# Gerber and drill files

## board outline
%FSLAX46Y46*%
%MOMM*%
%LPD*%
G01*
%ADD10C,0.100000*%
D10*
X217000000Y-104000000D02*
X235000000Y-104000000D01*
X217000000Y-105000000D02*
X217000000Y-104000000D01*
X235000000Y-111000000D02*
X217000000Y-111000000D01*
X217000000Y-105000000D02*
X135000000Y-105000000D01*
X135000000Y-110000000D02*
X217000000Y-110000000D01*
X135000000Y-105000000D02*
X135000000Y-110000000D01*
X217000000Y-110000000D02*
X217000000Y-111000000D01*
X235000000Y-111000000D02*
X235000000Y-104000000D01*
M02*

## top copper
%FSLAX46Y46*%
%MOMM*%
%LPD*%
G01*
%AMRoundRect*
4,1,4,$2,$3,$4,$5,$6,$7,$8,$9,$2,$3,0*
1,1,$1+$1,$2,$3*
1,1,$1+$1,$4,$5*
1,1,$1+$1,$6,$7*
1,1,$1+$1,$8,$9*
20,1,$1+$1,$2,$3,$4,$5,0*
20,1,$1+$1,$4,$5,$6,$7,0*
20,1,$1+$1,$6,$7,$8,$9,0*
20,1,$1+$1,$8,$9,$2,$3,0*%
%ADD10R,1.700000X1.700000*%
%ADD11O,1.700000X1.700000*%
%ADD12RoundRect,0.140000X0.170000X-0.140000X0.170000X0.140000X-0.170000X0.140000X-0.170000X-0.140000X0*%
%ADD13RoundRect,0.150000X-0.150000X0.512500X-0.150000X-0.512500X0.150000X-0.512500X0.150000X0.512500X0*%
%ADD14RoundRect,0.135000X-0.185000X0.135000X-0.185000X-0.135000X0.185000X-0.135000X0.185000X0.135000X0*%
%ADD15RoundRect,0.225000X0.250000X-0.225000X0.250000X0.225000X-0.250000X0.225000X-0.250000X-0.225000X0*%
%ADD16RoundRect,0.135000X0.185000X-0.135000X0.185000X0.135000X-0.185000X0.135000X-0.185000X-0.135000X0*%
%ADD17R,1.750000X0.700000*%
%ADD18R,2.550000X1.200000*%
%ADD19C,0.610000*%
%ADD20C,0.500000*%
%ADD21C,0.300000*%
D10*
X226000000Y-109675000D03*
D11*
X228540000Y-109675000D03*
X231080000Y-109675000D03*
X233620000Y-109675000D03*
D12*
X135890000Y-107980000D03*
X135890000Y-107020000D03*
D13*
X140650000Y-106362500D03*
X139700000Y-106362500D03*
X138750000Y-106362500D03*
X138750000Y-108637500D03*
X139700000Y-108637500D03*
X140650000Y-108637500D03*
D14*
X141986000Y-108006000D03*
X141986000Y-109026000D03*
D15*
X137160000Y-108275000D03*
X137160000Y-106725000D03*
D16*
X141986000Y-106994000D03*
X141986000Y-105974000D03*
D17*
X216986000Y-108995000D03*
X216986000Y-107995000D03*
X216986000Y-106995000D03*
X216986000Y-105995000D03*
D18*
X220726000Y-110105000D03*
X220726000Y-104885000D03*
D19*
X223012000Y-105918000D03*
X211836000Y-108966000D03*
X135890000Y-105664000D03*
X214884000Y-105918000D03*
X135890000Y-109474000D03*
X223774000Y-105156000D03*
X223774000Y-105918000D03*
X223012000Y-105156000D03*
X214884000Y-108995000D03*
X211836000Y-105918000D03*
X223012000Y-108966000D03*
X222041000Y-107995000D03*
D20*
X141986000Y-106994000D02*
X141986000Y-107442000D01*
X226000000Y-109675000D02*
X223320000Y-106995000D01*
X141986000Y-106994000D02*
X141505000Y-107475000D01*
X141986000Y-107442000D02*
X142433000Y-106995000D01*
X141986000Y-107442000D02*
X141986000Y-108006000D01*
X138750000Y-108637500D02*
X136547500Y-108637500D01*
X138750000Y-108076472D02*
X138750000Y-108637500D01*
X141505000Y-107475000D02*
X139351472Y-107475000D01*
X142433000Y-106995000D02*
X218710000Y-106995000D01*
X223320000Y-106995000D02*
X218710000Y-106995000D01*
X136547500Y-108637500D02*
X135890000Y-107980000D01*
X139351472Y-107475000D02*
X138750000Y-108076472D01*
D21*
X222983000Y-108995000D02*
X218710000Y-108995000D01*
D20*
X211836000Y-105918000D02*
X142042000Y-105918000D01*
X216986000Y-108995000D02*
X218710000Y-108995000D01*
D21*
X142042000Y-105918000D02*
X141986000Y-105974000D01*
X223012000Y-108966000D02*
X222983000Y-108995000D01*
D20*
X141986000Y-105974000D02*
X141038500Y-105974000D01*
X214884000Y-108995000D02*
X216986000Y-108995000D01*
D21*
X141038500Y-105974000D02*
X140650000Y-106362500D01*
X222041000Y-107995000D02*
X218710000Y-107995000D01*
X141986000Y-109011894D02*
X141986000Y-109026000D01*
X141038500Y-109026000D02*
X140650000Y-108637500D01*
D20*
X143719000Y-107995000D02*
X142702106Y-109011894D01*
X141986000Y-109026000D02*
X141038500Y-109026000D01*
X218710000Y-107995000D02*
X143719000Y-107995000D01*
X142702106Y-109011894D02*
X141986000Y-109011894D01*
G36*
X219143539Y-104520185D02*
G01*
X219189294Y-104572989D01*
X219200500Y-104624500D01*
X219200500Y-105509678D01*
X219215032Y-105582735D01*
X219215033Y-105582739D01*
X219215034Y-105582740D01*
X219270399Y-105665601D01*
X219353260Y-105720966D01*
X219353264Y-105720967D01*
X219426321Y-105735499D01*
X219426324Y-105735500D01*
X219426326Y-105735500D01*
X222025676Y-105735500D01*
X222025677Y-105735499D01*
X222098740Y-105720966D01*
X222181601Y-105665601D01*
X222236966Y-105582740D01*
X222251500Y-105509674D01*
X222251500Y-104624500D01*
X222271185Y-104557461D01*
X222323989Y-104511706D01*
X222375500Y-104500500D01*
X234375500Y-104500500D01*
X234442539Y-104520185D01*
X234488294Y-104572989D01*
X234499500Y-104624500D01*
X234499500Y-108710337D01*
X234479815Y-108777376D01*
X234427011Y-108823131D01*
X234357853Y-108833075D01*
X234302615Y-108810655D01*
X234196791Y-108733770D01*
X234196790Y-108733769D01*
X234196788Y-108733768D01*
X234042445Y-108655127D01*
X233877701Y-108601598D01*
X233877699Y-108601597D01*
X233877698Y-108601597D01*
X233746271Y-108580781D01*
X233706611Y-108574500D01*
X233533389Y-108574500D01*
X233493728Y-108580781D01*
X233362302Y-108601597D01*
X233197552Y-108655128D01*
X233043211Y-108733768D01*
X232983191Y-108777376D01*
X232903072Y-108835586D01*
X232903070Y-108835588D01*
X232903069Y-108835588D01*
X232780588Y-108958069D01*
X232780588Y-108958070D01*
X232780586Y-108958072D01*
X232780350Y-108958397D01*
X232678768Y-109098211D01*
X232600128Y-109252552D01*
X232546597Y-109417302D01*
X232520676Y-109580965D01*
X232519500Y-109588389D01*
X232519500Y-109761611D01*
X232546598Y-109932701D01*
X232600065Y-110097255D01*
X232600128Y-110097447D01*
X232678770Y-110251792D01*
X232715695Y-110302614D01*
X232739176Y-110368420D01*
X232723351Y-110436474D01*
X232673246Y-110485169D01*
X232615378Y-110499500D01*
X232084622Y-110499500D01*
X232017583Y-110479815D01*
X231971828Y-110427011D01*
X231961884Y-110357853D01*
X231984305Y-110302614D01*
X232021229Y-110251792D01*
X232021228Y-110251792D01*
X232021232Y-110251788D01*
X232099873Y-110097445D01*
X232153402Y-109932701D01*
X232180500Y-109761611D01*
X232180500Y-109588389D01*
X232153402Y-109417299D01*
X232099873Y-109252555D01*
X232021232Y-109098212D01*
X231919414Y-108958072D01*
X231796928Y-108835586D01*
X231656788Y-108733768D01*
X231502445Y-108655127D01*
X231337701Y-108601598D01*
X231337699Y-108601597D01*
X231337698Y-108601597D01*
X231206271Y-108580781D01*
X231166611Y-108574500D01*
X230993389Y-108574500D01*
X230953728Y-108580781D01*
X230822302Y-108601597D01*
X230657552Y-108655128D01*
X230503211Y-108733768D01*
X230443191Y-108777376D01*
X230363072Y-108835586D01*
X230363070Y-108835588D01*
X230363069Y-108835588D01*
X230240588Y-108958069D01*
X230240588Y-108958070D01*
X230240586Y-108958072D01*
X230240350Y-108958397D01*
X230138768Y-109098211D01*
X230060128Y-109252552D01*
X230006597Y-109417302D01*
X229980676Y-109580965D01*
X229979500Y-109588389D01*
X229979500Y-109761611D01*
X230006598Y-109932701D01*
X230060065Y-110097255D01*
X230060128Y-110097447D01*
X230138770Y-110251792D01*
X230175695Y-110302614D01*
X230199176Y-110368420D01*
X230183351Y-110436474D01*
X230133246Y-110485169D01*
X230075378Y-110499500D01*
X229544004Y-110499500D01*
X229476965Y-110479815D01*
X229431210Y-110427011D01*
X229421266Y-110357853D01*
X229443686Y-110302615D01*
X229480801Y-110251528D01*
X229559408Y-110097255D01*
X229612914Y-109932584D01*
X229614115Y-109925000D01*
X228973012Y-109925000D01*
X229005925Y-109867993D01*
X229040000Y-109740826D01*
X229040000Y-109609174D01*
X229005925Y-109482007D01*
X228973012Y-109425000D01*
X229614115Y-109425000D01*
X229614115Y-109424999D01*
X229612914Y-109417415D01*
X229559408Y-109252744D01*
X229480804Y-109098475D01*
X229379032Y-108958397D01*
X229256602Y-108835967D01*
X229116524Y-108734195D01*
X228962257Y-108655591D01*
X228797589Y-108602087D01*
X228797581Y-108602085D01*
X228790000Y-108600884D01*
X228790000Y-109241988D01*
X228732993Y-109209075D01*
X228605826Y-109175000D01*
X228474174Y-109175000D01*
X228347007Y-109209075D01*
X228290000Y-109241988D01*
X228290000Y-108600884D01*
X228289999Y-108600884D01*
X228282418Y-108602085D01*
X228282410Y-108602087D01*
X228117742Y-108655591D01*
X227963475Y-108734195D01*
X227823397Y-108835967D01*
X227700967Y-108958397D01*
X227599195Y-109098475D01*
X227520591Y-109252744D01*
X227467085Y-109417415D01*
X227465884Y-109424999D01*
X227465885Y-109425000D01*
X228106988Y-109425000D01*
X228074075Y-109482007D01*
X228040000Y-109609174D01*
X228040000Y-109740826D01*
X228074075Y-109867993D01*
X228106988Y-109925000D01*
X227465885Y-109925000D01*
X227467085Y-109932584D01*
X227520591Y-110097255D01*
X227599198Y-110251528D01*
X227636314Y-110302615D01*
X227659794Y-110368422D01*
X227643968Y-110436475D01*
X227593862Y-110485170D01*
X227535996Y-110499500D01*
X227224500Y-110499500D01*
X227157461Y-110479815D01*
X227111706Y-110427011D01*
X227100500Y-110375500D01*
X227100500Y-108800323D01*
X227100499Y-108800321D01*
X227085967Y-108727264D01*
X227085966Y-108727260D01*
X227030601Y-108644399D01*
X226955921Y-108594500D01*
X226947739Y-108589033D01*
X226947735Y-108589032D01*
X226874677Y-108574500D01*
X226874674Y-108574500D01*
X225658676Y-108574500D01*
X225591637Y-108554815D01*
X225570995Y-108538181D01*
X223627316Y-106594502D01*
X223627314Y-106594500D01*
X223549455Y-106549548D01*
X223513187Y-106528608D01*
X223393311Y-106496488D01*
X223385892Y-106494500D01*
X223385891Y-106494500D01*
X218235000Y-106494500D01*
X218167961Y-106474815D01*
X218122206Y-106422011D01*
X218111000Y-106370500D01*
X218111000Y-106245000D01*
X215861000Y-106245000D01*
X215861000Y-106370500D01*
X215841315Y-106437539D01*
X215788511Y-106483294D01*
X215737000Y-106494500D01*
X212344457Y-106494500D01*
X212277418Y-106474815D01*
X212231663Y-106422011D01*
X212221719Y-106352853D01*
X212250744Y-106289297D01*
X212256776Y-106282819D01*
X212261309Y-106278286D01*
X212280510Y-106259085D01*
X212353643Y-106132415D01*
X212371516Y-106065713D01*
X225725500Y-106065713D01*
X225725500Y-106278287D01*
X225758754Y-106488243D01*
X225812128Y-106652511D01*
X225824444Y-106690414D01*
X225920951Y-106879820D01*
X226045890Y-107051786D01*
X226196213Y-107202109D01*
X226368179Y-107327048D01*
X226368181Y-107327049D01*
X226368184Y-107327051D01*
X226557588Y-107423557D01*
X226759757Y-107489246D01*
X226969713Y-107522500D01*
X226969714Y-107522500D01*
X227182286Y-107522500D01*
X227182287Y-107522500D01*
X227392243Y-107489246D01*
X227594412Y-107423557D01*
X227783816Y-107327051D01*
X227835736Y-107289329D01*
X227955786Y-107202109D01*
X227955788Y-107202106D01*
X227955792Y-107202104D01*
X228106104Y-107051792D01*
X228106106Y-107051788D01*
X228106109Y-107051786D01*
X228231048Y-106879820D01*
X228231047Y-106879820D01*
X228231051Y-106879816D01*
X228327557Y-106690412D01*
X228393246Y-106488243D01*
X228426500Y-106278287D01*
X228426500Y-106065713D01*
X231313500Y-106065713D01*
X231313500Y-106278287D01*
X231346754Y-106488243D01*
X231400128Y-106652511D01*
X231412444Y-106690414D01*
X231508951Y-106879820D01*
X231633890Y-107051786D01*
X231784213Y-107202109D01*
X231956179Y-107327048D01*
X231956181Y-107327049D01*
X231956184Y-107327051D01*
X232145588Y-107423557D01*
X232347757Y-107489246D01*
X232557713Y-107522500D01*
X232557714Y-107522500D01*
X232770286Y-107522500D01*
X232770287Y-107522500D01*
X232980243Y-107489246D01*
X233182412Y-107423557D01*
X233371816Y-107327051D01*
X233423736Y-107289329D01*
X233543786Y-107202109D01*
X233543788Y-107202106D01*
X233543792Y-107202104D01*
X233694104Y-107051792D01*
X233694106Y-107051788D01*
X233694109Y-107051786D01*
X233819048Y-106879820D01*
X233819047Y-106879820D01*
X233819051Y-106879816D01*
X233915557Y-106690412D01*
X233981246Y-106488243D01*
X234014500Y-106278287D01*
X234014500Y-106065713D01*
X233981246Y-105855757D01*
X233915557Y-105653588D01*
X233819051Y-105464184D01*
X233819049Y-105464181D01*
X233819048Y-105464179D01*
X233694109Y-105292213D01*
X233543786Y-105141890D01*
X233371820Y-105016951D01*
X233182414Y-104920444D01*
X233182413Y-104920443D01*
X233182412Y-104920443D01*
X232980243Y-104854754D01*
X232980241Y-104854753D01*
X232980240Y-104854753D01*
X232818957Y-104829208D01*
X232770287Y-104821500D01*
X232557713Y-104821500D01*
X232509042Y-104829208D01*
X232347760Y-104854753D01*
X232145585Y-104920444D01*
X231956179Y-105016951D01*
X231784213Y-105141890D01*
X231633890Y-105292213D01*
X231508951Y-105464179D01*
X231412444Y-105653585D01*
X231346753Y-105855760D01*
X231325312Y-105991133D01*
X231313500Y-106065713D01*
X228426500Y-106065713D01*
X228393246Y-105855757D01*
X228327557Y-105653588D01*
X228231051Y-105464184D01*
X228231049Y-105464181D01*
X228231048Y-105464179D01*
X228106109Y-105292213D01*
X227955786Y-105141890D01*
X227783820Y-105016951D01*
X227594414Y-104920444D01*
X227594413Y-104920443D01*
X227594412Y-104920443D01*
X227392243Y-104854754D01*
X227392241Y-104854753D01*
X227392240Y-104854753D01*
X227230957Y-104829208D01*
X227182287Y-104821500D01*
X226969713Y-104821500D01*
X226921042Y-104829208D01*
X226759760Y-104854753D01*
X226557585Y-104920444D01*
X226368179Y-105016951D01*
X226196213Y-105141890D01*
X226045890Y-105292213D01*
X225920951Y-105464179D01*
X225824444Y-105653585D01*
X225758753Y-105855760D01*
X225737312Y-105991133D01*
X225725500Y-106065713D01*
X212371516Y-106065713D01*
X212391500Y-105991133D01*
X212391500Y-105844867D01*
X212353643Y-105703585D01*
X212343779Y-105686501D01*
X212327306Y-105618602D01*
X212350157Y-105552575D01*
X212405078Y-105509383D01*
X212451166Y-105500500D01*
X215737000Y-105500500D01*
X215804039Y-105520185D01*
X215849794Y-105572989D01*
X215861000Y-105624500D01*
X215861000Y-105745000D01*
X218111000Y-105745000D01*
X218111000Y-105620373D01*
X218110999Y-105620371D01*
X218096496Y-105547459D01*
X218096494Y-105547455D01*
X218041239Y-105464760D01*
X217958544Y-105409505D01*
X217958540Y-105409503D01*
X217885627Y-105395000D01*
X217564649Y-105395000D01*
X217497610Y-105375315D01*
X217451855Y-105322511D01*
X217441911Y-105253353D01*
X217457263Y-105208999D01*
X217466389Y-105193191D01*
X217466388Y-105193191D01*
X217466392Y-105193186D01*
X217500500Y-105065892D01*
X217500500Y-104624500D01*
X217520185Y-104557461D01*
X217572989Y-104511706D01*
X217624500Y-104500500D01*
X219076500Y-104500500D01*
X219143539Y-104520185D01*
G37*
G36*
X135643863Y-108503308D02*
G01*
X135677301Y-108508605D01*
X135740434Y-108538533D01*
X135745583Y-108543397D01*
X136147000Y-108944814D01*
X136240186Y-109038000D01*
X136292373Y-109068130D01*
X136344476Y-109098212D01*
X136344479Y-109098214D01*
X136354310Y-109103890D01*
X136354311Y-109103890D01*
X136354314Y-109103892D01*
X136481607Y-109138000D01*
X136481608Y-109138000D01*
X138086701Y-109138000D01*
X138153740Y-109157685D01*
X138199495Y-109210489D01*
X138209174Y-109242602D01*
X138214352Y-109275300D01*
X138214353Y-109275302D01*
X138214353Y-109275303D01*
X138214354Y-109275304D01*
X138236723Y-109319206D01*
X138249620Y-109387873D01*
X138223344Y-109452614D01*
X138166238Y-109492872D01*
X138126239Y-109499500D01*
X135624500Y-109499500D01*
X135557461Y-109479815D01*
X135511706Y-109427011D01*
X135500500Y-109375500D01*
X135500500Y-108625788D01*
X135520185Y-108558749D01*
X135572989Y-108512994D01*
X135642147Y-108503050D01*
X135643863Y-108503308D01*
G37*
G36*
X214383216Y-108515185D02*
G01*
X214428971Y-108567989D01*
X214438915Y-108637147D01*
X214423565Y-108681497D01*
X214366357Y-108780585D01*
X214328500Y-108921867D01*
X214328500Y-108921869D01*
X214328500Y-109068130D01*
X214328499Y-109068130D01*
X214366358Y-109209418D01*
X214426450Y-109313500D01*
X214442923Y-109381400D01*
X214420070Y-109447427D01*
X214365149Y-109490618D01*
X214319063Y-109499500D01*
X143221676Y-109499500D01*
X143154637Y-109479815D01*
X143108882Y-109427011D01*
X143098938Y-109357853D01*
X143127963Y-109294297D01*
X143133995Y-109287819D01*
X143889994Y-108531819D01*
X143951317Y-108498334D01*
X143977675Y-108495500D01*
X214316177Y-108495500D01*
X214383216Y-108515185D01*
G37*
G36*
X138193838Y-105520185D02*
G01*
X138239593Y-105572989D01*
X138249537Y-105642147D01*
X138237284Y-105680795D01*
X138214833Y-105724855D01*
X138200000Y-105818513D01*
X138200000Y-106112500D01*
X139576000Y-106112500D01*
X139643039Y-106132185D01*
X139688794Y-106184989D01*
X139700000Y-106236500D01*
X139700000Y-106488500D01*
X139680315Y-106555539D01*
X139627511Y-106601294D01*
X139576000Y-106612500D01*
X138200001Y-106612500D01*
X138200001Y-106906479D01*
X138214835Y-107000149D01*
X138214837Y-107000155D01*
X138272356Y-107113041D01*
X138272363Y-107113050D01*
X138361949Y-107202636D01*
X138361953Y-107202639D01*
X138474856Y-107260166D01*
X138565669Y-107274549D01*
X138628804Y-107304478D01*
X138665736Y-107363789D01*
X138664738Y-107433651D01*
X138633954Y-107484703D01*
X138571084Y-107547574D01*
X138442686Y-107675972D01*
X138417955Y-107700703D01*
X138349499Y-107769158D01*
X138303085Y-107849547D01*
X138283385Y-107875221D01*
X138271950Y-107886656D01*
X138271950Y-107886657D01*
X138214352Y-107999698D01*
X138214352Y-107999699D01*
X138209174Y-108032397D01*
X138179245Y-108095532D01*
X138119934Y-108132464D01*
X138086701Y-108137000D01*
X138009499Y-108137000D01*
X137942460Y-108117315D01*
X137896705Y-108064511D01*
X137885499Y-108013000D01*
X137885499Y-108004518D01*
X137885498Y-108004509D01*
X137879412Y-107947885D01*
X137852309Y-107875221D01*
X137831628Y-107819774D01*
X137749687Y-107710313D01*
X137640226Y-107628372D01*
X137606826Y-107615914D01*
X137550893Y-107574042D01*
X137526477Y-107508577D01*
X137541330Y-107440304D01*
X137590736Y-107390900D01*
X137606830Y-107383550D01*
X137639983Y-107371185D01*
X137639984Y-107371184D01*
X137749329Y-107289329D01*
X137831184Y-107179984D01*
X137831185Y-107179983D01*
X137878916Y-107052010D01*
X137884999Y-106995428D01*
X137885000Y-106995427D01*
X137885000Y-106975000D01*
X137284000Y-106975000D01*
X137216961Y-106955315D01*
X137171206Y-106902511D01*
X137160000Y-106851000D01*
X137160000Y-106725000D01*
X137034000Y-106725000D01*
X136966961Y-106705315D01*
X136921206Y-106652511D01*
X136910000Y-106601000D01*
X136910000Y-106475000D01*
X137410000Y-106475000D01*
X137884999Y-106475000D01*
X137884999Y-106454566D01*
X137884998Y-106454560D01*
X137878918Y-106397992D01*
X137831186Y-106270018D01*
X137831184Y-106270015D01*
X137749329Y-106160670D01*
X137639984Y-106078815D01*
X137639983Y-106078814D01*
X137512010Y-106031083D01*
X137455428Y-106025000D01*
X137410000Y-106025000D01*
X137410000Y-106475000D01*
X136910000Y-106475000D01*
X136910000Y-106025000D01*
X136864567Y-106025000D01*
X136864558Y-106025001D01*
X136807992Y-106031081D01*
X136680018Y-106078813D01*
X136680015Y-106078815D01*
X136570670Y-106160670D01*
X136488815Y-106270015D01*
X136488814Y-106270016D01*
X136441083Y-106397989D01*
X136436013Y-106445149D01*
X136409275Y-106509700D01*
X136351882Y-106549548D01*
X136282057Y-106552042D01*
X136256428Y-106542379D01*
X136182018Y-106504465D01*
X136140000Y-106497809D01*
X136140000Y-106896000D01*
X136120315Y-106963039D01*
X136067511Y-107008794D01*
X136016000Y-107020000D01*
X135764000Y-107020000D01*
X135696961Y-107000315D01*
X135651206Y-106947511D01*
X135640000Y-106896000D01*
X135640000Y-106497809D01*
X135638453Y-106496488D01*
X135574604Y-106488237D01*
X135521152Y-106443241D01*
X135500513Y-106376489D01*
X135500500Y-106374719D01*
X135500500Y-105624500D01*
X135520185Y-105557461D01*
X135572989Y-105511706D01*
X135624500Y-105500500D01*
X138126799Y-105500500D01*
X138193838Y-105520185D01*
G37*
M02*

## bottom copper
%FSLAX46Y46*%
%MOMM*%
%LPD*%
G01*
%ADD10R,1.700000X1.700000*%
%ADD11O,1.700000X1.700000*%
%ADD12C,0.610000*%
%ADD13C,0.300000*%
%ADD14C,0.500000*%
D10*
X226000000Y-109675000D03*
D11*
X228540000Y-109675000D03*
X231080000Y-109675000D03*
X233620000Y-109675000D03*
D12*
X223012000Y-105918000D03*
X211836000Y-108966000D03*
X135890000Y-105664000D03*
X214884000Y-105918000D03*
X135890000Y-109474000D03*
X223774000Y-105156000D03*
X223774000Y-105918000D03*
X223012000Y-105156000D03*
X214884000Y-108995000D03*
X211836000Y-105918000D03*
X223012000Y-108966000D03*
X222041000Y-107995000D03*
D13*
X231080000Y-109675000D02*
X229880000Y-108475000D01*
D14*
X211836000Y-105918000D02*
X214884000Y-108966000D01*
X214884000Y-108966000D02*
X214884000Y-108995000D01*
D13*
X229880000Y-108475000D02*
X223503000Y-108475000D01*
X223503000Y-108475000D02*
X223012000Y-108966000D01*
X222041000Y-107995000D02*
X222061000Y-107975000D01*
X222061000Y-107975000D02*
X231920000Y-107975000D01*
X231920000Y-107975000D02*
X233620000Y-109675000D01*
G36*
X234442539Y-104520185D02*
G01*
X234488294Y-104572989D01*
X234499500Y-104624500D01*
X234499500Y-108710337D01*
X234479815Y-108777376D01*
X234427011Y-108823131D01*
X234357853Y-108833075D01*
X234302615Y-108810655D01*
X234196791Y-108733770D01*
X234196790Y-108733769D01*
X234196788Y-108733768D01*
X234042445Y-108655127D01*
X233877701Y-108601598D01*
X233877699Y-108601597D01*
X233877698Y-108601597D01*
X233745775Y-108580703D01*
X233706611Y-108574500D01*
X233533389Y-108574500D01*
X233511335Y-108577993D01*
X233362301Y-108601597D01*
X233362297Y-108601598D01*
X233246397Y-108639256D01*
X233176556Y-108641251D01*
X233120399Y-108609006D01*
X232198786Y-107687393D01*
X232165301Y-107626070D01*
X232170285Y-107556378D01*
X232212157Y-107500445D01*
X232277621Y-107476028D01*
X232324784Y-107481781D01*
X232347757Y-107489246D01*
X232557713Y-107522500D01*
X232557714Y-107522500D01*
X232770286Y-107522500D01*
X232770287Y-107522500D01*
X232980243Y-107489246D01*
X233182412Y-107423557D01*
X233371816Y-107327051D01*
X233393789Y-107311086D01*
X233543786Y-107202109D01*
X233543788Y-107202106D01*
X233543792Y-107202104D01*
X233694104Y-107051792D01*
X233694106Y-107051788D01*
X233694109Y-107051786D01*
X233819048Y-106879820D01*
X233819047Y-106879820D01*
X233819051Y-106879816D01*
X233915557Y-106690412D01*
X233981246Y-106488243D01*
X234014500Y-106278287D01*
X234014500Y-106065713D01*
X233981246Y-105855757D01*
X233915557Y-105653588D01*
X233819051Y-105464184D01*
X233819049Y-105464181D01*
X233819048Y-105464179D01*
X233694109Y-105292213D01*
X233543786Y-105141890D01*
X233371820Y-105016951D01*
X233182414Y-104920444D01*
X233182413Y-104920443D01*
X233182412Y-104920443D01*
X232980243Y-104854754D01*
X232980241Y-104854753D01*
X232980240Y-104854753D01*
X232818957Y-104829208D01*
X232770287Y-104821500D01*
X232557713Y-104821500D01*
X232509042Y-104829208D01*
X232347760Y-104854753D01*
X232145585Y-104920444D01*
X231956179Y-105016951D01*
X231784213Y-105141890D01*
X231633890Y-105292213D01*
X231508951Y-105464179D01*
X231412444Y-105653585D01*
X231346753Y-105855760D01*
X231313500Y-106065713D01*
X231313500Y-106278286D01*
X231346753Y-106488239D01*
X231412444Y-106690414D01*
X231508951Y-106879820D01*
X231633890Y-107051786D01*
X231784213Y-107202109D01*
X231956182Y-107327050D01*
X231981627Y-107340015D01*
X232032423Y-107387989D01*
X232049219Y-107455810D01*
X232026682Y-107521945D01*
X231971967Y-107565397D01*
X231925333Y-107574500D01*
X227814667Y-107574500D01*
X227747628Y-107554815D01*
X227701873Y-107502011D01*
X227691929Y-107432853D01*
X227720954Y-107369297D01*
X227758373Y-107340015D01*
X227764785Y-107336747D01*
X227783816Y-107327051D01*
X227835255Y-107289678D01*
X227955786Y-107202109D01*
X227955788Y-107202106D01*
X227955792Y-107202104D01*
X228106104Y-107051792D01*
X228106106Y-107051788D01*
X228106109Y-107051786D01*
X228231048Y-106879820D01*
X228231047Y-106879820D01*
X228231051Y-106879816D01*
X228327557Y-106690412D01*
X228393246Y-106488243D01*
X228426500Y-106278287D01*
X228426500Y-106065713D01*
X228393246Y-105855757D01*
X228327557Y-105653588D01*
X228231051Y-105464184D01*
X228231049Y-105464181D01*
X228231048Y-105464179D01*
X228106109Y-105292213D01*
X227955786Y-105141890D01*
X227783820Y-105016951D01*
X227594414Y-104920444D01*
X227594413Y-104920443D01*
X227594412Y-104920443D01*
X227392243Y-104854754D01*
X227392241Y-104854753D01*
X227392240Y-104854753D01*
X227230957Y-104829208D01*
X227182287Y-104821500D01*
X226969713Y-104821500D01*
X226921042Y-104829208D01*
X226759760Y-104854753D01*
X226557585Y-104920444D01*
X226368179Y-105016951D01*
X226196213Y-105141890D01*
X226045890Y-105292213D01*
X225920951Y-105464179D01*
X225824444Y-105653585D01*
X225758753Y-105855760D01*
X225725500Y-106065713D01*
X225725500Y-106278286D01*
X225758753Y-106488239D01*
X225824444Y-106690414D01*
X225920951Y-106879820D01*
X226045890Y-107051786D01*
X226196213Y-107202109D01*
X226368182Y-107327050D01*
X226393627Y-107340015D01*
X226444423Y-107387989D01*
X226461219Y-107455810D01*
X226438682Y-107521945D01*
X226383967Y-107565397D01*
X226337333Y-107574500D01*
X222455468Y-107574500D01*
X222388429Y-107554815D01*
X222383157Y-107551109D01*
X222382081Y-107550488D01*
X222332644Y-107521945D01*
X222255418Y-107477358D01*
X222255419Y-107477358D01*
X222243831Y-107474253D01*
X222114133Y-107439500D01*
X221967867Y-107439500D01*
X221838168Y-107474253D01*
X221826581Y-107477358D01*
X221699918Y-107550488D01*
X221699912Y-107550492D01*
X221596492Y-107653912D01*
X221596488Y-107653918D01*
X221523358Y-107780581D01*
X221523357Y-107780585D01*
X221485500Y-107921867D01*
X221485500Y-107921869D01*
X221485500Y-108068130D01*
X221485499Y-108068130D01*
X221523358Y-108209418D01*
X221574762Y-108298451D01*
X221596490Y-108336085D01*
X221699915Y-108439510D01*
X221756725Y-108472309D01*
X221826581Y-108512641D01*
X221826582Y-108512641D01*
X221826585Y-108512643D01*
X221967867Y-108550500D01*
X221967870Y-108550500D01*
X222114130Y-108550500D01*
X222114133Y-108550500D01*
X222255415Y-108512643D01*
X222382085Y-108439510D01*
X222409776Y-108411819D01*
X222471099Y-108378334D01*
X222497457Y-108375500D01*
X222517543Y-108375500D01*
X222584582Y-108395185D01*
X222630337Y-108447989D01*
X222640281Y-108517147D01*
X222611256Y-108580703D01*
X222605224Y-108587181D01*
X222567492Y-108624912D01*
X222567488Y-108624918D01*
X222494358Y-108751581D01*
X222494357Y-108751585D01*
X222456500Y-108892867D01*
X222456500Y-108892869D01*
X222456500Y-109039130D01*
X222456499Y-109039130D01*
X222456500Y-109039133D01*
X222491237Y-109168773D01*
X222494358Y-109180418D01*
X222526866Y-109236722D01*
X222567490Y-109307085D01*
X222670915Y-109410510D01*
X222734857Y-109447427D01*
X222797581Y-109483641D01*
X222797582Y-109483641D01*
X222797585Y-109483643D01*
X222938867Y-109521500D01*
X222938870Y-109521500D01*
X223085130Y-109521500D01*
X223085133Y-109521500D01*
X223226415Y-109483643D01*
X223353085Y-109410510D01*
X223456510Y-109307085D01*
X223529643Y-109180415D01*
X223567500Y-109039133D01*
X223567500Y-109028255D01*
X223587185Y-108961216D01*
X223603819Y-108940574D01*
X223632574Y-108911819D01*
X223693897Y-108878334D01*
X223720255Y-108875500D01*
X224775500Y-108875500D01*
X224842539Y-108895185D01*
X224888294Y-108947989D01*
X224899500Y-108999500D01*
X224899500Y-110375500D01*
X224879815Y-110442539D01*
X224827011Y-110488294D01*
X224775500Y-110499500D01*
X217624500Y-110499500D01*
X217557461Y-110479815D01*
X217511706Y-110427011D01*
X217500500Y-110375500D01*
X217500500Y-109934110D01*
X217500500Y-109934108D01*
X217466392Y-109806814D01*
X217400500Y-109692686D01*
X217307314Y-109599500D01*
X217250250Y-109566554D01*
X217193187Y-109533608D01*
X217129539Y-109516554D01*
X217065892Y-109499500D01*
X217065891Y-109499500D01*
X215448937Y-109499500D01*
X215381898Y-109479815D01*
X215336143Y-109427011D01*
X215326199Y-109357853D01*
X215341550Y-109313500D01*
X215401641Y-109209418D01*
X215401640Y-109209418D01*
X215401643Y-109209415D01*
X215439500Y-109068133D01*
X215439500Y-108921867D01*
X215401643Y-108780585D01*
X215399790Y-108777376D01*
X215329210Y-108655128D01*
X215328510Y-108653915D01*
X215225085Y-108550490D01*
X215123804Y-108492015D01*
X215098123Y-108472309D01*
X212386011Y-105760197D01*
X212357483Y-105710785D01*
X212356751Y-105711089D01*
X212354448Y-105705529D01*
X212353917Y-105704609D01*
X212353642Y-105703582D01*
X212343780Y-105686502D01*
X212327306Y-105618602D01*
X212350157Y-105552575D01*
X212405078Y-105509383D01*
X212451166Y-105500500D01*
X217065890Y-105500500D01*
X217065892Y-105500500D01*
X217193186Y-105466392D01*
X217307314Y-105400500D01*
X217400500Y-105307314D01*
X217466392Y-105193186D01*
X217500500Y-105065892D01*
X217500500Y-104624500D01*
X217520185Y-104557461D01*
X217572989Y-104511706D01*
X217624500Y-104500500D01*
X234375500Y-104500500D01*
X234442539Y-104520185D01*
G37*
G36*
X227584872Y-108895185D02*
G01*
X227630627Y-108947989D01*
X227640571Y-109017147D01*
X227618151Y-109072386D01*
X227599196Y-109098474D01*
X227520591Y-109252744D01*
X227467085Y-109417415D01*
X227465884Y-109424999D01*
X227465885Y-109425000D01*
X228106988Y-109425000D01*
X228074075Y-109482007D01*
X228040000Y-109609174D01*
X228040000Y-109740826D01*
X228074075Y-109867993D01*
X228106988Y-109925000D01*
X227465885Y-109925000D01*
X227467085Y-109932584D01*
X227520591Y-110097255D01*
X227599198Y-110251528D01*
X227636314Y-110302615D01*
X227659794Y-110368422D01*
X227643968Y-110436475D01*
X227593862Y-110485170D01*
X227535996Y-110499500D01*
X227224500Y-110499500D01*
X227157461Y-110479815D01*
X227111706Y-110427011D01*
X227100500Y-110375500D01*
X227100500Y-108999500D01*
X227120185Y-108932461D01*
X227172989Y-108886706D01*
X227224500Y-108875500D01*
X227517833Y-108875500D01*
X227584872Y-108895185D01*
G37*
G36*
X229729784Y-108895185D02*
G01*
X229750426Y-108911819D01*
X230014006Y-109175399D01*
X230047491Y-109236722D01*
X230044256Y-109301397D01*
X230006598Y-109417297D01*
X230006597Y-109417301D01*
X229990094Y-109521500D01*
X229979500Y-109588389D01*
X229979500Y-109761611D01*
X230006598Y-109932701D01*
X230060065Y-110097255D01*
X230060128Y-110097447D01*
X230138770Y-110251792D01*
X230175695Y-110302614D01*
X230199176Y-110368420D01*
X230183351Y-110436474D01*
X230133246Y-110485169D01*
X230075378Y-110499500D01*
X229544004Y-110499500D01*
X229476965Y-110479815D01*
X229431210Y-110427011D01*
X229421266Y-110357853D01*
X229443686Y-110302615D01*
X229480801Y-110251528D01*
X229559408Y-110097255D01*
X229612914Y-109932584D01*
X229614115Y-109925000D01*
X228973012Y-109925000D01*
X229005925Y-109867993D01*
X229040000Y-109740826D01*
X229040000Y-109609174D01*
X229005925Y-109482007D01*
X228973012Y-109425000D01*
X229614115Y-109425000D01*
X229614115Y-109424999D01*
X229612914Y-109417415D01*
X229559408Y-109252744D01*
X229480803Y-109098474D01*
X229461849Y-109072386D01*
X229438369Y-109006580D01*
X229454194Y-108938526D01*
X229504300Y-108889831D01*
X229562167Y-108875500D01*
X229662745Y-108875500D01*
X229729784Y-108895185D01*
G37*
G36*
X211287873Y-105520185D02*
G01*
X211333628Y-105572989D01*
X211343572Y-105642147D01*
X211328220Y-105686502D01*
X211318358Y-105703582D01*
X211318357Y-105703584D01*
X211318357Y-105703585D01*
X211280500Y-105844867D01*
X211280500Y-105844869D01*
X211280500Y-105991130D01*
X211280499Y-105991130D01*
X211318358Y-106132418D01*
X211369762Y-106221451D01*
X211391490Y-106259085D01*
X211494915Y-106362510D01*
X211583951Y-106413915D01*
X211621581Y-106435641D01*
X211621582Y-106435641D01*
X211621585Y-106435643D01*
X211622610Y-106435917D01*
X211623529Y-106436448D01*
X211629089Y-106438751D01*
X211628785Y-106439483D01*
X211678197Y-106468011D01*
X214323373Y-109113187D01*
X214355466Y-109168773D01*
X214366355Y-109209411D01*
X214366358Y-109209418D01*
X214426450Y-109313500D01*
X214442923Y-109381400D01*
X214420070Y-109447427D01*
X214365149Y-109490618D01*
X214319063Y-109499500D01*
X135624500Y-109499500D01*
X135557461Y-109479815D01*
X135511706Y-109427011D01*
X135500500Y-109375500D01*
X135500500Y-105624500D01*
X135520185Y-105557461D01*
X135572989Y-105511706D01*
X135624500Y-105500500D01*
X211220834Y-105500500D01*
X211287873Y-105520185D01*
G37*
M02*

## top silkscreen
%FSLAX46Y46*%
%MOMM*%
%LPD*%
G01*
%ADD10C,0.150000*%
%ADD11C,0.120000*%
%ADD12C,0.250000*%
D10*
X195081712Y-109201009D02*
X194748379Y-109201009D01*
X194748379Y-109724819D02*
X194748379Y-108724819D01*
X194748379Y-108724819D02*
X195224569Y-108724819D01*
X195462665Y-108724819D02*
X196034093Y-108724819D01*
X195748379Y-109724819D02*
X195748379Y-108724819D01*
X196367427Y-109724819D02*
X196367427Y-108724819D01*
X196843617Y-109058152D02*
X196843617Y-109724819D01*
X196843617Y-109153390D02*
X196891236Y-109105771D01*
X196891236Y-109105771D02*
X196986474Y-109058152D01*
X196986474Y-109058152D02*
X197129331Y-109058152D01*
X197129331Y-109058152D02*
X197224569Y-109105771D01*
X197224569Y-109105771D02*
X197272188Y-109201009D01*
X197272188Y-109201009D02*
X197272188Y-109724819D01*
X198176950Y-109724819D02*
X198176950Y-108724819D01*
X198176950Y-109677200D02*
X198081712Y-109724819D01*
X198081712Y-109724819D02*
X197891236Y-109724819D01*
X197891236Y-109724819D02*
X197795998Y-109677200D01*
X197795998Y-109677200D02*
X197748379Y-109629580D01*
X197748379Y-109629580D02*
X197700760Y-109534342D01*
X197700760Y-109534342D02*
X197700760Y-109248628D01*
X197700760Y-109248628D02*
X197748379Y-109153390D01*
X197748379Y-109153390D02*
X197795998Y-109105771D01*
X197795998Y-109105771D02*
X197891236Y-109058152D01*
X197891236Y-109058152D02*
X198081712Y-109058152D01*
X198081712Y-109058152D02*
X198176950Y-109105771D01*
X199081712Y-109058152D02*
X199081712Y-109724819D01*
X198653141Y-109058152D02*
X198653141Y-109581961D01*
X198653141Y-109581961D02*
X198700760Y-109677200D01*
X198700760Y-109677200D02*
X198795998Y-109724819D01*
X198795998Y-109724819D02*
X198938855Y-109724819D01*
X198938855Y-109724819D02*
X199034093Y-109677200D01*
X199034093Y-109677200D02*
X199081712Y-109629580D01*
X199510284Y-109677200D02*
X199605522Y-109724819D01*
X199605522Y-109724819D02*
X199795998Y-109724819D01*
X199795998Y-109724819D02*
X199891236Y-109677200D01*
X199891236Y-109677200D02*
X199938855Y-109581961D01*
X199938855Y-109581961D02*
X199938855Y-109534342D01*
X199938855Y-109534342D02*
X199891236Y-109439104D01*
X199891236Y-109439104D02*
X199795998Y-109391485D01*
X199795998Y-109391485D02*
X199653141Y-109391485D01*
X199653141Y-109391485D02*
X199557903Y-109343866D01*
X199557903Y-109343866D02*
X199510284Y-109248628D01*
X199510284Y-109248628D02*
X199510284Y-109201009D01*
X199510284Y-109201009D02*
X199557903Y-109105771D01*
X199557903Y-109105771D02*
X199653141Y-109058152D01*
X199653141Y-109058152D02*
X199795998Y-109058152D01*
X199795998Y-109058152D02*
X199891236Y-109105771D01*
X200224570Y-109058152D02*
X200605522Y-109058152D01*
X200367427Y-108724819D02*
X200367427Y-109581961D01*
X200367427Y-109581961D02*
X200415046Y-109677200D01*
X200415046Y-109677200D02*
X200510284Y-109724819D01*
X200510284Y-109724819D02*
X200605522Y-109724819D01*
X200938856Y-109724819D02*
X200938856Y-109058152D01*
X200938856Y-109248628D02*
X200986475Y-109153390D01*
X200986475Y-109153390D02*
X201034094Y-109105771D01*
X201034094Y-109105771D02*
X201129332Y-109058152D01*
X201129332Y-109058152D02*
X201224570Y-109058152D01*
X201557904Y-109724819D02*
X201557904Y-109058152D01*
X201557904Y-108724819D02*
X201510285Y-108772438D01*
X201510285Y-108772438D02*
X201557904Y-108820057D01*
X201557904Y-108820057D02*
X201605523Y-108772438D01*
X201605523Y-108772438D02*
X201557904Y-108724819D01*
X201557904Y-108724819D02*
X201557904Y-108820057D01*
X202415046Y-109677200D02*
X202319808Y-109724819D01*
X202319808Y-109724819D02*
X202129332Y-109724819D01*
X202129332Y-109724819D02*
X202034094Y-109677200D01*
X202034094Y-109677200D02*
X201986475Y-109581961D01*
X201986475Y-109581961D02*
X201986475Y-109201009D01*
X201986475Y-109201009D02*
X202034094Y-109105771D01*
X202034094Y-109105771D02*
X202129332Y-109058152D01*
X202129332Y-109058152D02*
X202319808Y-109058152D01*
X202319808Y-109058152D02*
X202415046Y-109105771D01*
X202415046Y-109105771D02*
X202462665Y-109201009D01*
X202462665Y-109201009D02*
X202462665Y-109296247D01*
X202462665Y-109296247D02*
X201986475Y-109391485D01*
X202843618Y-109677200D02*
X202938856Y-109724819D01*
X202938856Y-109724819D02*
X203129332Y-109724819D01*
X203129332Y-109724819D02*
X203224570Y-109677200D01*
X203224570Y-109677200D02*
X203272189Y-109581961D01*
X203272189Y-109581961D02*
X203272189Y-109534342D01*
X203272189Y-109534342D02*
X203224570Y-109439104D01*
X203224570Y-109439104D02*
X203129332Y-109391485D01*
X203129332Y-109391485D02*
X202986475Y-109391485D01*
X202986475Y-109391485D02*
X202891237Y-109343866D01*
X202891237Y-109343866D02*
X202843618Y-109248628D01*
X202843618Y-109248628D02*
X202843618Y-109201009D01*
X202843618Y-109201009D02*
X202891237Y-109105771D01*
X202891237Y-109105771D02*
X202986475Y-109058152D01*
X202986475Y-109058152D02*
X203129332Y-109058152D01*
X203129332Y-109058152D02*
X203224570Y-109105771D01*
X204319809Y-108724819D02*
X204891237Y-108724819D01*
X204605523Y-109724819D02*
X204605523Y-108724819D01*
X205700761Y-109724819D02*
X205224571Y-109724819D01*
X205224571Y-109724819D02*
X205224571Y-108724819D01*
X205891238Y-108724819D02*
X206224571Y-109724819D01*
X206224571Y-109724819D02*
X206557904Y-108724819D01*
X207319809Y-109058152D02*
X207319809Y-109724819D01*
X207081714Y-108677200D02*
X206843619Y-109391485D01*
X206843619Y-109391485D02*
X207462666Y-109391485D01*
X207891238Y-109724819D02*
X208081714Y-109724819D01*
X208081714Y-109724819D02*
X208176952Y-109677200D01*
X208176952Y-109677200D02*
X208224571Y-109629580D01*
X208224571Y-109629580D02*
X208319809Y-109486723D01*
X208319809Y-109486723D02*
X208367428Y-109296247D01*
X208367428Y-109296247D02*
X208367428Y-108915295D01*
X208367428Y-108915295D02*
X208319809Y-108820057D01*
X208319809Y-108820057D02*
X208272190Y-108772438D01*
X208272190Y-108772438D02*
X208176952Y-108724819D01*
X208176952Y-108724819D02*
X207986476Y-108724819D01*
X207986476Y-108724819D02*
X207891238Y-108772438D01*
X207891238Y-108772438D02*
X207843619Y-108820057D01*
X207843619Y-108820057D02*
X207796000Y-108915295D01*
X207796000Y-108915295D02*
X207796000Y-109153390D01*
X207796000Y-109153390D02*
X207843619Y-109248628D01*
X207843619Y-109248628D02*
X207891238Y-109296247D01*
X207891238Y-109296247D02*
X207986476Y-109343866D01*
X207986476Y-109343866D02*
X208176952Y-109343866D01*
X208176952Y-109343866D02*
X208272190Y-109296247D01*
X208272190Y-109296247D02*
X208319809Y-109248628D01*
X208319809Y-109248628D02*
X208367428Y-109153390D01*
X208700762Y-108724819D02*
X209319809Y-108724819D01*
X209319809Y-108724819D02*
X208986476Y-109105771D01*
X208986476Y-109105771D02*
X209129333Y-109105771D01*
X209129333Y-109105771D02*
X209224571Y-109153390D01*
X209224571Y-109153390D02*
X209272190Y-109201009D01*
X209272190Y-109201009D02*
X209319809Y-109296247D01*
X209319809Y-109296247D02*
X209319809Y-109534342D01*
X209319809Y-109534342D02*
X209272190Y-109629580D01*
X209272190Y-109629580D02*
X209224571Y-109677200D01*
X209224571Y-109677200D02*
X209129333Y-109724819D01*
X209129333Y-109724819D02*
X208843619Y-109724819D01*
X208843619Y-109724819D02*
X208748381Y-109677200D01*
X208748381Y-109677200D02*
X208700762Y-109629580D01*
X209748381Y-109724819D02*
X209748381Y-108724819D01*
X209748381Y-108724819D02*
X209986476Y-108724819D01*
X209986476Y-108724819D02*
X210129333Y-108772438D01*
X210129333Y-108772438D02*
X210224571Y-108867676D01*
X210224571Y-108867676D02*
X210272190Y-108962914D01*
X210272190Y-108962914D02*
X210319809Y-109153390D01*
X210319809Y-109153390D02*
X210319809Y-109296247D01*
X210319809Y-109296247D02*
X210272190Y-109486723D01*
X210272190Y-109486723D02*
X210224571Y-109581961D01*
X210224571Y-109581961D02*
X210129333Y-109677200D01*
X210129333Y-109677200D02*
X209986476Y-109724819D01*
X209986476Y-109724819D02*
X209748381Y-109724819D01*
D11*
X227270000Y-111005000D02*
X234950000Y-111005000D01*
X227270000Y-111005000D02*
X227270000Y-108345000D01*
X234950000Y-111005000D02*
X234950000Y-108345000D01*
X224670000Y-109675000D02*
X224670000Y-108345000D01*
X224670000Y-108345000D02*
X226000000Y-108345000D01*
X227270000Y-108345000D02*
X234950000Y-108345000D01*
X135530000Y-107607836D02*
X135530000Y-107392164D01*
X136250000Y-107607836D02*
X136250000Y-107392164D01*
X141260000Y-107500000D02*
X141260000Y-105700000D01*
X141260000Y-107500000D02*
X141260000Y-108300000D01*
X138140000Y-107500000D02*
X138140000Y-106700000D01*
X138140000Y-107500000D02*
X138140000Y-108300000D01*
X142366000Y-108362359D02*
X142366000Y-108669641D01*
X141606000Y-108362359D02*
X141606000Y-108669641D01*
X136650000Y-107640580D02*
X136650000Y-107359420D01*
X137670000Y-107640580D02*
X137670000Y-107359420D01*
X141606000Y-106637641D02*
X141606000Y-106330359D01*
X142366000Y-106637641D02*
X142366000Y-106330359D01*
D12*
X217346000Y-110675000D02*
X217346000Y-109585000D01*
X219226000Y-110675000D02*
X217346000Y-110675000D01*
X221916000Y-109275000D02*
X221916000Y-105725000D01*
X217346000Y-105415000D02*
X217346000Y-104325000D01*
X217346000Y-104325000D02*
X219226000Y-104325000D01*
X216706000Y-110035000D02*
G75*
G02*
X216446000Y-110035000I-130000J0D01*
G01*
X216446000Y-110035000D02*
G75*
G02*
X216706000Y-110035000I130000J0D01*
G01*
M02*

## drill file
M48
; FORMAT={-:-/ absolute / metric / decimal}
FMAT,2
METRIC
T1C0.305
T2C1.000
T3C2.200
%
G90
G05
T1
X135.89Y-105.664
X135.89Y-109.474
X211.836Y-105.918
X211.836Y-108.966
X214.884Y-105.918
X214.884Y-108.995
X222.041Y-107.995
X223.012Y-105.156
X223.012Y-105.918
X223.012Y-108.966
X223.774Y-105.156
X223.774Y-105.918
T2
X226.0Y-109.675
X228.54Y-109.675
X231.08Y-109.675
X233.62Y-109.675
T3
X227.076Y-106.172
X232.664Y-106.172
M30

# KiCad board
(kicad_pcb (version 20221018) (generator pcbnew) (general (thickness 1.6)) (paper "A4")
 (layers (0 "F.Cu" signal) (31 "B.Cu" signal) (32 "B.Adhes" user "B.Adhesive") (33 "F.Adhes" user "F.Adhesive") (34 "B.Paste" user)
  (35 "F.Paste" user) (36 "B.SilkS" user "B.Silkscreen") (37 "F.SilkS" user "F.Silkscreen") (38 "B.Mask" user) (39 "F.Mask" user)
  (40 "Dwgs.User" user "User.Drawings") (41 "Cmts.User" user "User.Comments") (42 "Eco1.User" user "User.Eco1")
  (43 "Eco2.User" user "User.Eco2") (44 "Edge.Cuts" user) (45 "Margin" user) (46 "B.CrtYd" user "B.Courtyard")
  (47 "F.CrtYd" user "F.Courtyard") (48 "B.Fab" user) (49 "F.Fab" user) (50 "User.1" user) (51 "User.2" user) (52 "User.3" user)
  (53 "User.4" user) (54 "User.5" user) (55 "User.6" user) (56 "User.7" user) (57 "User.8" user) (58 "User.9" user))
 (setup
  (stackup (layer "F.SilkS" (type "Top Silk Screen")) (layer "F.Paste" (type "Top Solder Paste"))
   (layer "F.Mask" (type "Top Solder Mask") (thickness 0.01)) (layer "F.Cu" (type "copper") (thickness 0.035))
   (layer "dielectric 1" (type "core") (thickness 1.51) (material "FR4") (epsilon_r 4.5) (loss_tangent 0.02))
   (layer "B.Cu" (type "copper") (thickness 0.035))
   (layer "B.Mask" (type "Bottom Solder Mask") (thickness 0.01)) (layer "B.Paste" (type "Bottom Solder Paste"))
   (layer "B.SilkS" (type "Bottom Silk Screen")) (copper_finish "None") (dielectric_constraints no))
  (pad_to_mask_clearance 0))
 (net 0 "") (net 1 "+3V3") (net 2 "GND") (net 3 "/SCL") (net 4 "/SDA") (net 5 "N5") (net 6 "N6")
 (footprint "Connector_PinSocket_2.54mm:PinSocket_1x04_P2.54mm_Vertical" (layer "F.Cu") (at 226 109.675 90)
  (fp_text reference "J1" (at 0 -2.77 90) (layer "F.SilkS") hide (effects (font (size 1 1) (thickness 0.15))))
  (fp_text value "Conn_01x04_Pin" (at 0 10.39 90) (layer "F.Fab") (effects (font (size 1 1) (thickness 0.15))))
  (fp_line (start -1.33 1.27) (end -1.33 8.95) (stroke (width 0.12) (type solid)) (layer "F.SilkS"))
  (fp_line (start -1.33 1.27) (end 1.33 1.27) (stroke (width 0.12) (type solid)) (layer "F.SilkS"))
  (fp_line (start -1.33 8.95) (end 1.33 8.95) (stroke (width 0.12) (type solid)) (layer "F.SilkS"))
  (fp_line (start 0 -1.33) (end 1.33 -1.33) (stroke (width 0.12) (type solid)) (layer "F.SilkS"))
  (fp_line (start 1.33 -1.33) (end 1.33 0) (stroke (width 0.12) (type solid)) (layer "F.SilkS"))
  (fp_line (start 1.33 1.27) (end 1.33 8.95) (stroke (width 0.12) (type solid)) (layer "F.SilkS"))
  (pad "1" thru_hole rect (at 0 0 90) (size 1.7 1.7) (drill 1) (layers "*.Cu" "*.Mask") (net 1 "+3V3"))
  (pad "2" thru_hole oval (at 0 2.54 90) (size 1.7 1.7) (drill 1) (layers "*.Cu" "*.Mask") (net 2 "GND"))
  (pad "3" thru_hole oval (at 0 5.08 90) (size 1.7 1.7) (drill 1) (layers "*.Cu" "*.Mask") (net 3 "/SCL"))
  (pad "4" thru_hole oval (at 0 7.62 90) (size 1.7 1.7) (drill 1) (layers "*.Cu" "*.Mask") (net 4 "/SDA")))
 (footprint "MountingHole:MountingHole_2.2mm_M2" (layer "F.Cu") (at 232.664 106.172)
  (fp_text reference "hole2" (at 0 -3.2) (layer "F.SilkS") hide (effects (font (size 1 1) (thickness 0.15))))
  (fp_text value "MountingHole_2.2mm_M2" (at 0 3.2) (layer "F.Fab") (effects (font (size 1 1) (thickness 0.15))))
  (pad "" np_thru_hole circle (at 0 0) (size 2.2 2.2) (drill 2.2) (layers "*.Cu" "*.Mask")))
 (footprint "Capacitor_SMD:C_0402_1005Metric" (layer "F.Cu") (at 135.89 107.5 90)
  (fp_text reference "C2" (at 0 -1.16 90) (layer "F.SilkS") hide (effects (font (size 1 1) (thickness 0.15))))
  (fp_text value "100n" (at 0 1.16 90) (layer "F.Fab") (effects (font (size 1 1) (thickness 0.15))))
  (fp_line (start -0.107836 -0.36) (end 0.107836 -0.36) (stroke (width 0.12) (type solid)) (layer "F.SilkS"))
  (fp_line (start -0.107836 0.36) (end 0.107836 0.36) (stroke (width 0.12) (type solid)) (layer "F.SilkS"))
  (pad "1" smd roundrect (at -0.48 0 90) (size 0.56 0.62) (layers "F.Cu" "F.Paste" "F.Mask") (roundrect_rratio 0.25) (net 1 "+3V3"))
  (pad "2" smd roundrect (at 0.48 0 90) (size 0.56 0.62) (layers "F.Cu" "F.Paste" "F.Mask") (roundrect_rratio 0.25) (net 2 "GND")))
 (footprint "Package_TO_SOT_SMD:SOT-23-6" (layer "F.Cu") (at 139.7 107.5 -90)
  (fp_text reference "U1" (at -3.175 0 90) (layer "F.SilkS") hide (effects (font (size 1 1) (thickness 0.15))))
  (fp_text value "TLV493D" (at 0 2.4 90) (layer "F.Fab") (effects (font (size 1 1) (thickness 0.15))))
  (fp_line (start 0 -1.56) (end -1.8 -1.56) (stroke (width 0.12) (type solid)) (layer "F.SilkS"))
  (fp_line (start 0 -1.56) (end 0.8 -1.56) (stroke (width 0.12) (type solid)) (layer "F.SilkS"))
  (fp_line (start 0 1.56) (end -0.8 1.56) (stroke (width 0.12) (type solid)) (layer "F.SilkS"))
  (fp_line (start 0 1.56) (end 0.8 1.56) (stroke (width 0.12) (type solid)) (layer "F.SilkS"))
  (pad "1" smd roundrect (at -1.1375 -0.95 270) (size 1.325 0.6) (layers "F.Cu" "F.Paste" "F.Mask") (roundrect_rratio 0.25) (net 3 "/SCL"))
  (pad "2" smd roundrect (at -1.1375 0 270) (size 1.325 0.6) (layers "F.Cu" "F.Paste" "F.Mask") (roundrect_rratio 0.25) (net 2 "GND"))
  (pad "3" smd roundrect (at -1.1375 0.95 270) (size 1.325 0.6) (layers "F.Cu" "F.Paste" "F.Mask") (roundrect_rratio 0.25) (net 2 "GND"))
  (pad "4" smd roundrect (at 1.1375 0.95 270) (size 1.325 0.6) (layers "F.Cu" "F.Paste" "F.Mask") (roundrect_rratio 0.25) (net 1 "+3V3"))
  (pad "5" smd roundrect (at 1.1375 0 270) (size 1.325 0.6) (layers "F.Cu" "F.Paste" "F.Mask") (roundrect_rratio 0.25) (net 2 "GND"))
  (pad "6" smd roundrect (at 1.1375 -0.95 270) (size 1.325 0.6) (layers "F.Cu" "F.Paste" "F.Mask") (roundrect_rratio 0.25) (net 4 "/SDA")))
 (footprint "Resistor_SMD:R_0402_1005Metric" (layer "F.Cu") (at 141.986 108.516 -90)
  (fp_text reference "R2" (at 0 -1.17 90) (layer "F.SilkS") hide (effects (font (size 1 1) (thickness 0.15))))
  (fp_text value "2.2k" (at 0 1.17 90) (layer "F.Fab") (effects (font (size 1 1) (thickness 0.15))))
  (fp_line (start -0.153641 -0.38) (end 0.153641 -0.38) (stroke (width 0.12) (type solid)) (layer "F.SilkS"))
  (fp_line (start -0.153641 0.38) (end 0.153641 0.38) (stroke (width 0.12) (type solid)) (layer "F.SilkS"))
  (pad "1" smd roundrect (at -0.51 0 270) (size 0.54 0.64) (layers "F.Cu" "F.Paste" "F.Mask") (roundrect_rratio 0.25) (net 1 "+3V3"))
  (pad "2" smd roundrect (at 0.51 0 270) (size 0.54 0.64) (layers "F.Cu" "F.Paste" "F.Mask") (roundrect_rratio 0.25) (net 4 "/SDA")))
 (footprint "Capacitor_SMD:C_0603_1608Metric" (layer "F.Cu") (at 137.16 107.5 90)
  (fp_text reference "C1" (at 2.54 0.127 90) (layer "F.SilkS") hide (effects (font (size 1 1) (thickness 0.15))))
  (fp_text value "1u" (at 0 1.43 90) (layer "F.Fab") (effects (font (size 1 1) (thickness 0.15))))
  (fp_line (start -0.14058 -0.51) (end 0.14058 -0.51) (stroke (width 0.12) (type solid)) (layer "F.SilkS"))
  (fp_line (start -0.14058 0.51) (end 0.14058 0.51) (stroke (width 0.12) (type solid)) (layer "F.SilkS"))
  (pad "1" smd roundrect (at -0.775 0 90) (size 0.9 0.95) (layers "F.Cu" "F.Paste" "F.Mask") (roundrect_rratio 0.25) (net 1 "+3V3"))
  (pad "2" smd roundrect (at 0.775 0 90) (size 0.9 0.95) (layers "F.Cu" "F.Paste" "F.Mask") (roundrect_rratio 0.25) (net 2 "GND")))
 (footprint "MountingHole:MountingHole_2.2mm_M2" (layer "F.Cu") (at 227.076 106.172)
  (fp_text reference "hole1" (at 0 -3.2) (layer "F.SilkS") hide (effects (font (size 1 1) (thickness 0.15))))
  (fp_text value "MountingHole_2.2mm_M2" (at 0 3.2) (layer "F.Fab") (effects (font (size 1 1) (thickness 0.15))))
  (pad "" np_thru_hole circle (at 0 0) (size 2.2 2.2) (drill 2.2) (layers "*.Cu" "*.Mask")))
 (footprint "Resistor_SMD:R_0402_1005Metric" (layer "F.Cu") (at 141.986 106.484 90)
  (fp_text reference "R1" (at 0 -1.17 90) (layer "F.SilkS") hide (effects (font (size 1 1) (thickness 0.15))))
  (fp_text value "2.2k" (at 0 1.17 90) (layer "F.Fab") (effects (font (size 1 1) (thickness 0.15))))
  (fp_line (start -0.153641 -0.38) (end 0.153641 -0.38) (stroke (width 0.12) (type solid)) (layer "F.SilkS"))
  (fp_line (start -0.153641 0.38) (end 0.153641 0.38) (stroke (width 0.12) (type solid)) (layer "F.SilkS"))
  (pad "1" smd roundrect (at -0.51 0 90) (size 0.54 0.64) (layers "F.Cu" "F.Paste" "F.Mask") (roundrect_rratio 0.25) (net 1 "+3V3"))
  (pad "2" smd roundrect (at 0.51 0 90) (size 0.54 0.64) (layers "F.Cu" "F.Paste" "F.Mask") (roundrect_rratio 0.25) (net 3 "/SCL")))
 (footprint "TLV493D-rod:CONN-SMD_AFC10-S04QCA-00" (layer "F.Cu") (at 218.856 107.495 90)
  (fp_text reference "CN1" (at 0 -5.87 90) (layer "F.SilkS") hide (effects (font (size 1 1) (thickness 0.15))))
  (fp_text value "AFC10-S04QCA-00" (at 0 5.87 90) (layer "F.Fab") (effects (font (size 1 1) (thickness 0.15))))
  (fp_line (start -3.18 -1.51) (end -2.09 -1.51) (stroke (width 0.25) (type solid)) (layer "F.SilkS"))
  (fp_line (start -3.18 0.37) (end -3.18 -1.51) (stroke (width 0.25) (type solid)) (layer "F.SilkS"))
  (fp_line (start -1.78 3.06) (end 1.77 3.06) (stroke (width 0.25) (type solid)) (layer "F.SilkS"))
  (fp_line (start 2.08 -1.51) (end 3.17 -1.51) (stroke (width 0.25) (type solid)) (layer "F.SilkS"))
  (fp_line (start 3.17 -1.51) (end 3.17 0.37) (stroke (width 0.25) (type solid)) (layer "F.SilkS"))
  (fp_circle (center -2.54 -2.28) (end -2.41 -2.28) (stroke (width 0.25) (type solid)) (fill none) (layer "F.SilkS"))
  (pad "1" smd rect (at -1.5 -1.87 90) (size 0.7 1.75) (layers "F.Cu" "F.Paste" "F.Mask") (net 3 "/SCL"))
  (pad "2" smd rect (at -0.5 -1.87 90) (size 0.7 1.75) (layers "F.Cu" "F.Paste" "F.Mask") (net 4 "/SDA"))
  (pad "3" smd rect (at 0.5 -1.87 90) (size 0.7 1.75) (layers "F.Cu" "F.Paste" "F.Mask") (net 1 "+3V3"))
  (pad "4" smd rect (at 1.5 -1.87 90) (size 0.7 1.75) (layers "F.Cu" "F.Paste" "F.Mask") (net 2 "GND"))
  (pad "5" smd rect (at -2.61 1.87 90) (size 1.2 2.55) (layers "F.Cu" "F.Paste" "F.Mask") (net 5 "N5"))
  (pad "6" smd rect (at 2.61 1.87 90) (size 1.2 2.55) (layers "F.Cu" "F.Paste" "F.Mask") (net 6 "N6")))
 (gr_line (start 217 104) (end 235 104) (stroke (width 0.1) (type default)) (layer "Edge.Cuts"))
 (gr_line (start 217 105) (end 217 104) (stroke (width 0.1) (type default)) (layer "Edge.Cuts"))
 (gr_line (start 235 111) (end 217 111) (stroke (width 0.1) (type default)) (layer "Edge.Cuts"))
 (gr_line (start 217 105) (end 135 105) (stroke (width 0.1) (type default)) (layer "Edge.Cuts"))
 (gr_line (start 135 110) (end 217 110) (stroke (width 0.1) (type default)) (layer "Edge.Cuts"))
 (gr_line (start 135 105) (end 135 110) (stroke (width 0.1) (type default)) (layer "Edge.Cuts"))
 (gr_line (start 217 110) (end 217 111) (stroke (width 0.1) (type default)) (layer "Edge.Cuts"))
 (gr_line (start 235 111) (end 235 104) (stroke (width 0.1) (type default)) (layer "Edge.Cuts"))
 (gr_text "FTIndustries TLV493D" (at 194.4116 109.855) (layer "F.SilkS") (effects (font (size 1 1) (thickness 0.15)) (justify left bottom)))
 (segment (start 141.986 106.994) (end 141.986 107.442) (width 0.5) (layer "F.Cu") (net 1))
 (segment (start 226 109.675) (end 223.32 106.995) (width 0.5) (layer "F.Cu") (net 1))
 (segment (start 141.986 106.994) (end 141.505 107.475) (width 0.5) (layer "F.Cu") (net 1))
 (segment (start 141.986 107.442) (end 142.433 106.995) (width 0.5) (layer "F.Cu") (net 1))
 (segment (start 141.986 107.442) (end 141.986 108.006) (width 0.5) (layer "F.Cu") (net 1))
 (segment (start 138.75 108.6375) (end 136.5475 108.6375) (width 0.5) (layer "F.Cu") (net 1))
 (segment (start 138.75 108.076472) (end 138.75 108.6375) (width 0.5) (layer "F.Cu") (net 1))
 (segment (start 141.505 107.475) (end 139.351472 107.475) (width 0.5) (layer "F.Cu") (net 1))
 (segment (start 142.433 106.995) (end 218.71 106.995) (width 0.5) (layer "F.Cu") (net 1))
 (segment (start 223.32 106.995) (end 218.71 106.995) (width 0.5) (layer "F.Cu") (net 1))
 (segment (start 136.5475 108.6375) (end 135.89 107.98) (width 0.5) (layer "F.Cu") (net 1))
 (segment (start 139.351472 107.475) (end 138.75 108.076472) (width 0.5) (layer "F.Cu") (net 1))
 (via (at 223.012 105.918) (size 0.61) (drill 0.305) (layers "F.Cu" "B.Cu") (free) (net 2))
 (via (at 211.836 108.966) (size 0.61) (drill 0.305) (layers "F.Cu" "B.Cu") (free) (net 2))
 (via (at 135.89 105.664) (size 0.61) (drill 0.305) (layers "F.Cu" "B.Cu") (free) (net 2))
 (via (at 214.884 105.918) (size 0.61) (drill 0.305) (layers "F.Cu" "B.Cu") (free) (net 2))
 (via (at 135.89 109.474) (size 0.61) (drill 0.305) (layers "F.Cu" "B.Cu") (free) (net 2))
 (via (at 223.774 105.156) (size 0.61) (drill 0.305) (layers "F.Cu" "B.Cu") (free) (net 2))
 (via (at 223.774 105.918) (size 0.61) (drill 0.305) (layers "F.Cu" "B.Cu") (free) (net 2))
 (via (at 223.012 105.156) (size 0.61) (drill 0.305) (layers "F.Cu" "B.Cu") (free) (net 2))
 (segment (start 222.983 108.995) (end 218.71 108.995) (width 0.3) (layer "F.Cu") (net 3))
 (segment (start 211.836 105.918) (end 142.042 105.918) (width 0.5) (layer "F.Cu") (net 3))
 (segment (start 216.986 108.995) (end 218.71 108.995) (width 0.5) (layer "F.Cu") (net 3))
 (segment (start 142.042 105.918) (end 141.986 105.974) (width 0.3) (layer "F.Cu") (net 3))
 (segment (start 223.012 108.966) (end 222.983 108.995) (width 0.3) (layer "F.Cu") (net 3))
 (segment (start 141.986 105.974) (end 141.0385 105.974) (width 0.5) (layer "F.Cu") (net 3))
 (segment (start 214.884 108.995) (end 216.986 108.995) (width 0.5) (layer "F.Cu") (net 3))
 (segment (start 141.0385 105.974) (end 140.65 106.3625) (width 0.3) (layer "F.Cu") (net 3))
 (via (at 214.884 108.995) (size 0.61) (drill 0.305) (layers "F.Cu" "B.Cu") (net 3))
 (via (at 211.836 105.918) (size 0.61) (drill 0.305) (layers "F.Cu" "B.Cu") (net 3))
 (via (at 223.012 108.966) (size 0.61) (drill 0.305) (layers "F.Cu" "B.Cu") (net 3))
 (segment (start 231.08 109.675) (end 229.88 108.475) (width 0.3) (layer "B.Cu") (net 3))
 (segment (start 211.836 105.918) (end 214.884 108.966) (width 0.5) (layer "B.Cu") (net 3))
 (segment (start 214.884 108.966) (end 214.884 108.995) (width 0.5) (layer "B.Cu") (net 3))
 (segment (start 229.88 108.475) (end 223.503 108.475) (width 0.3) (layer "B.Cu") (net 3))
 (segment (start 223.503 108.475) (end 223.012 108.966) (width 0.3) (layer "B.Cu") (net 3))
 (segment (start 222.041 107.995) (end 218.71 107.995) (width 0.3) (layer "F.Cu") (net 4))
 (segment (start 141.986 109.011894) (end 141.986 109.026) (width 0.3) (layer "F.Cu") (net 4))
 (segment (start 141.0385 109.026) (end 140.65 108.6375) (width 0.3) (layer "F.Cu") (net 4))
 (segment (start 143.719 107.995) (end 142.702106 109.011894) (width 0.5) (layer "F.Cu") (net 4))
 (segment (start 141.986 109.026) (end 141.0385 109.026) (width 0.5) (layer "F.Cu") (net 4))
 (segment (start 218.71 107.995) (end 143.719 107.995) (width 0.5) (layer "F.Cu") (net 4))
 (segment (start 142.702106 109.011894) (end 141.986 109.011894) (width 0.5) (layer "F.Cu") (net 4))
 (via (at 222.041 107.995) (size 0.61) (drill 0.305) (layers "F.Cu" "B.Cu") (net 4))
 (segment (start 222.041 107.995) (end 222.061 107.975) (width 0.3) (layer "B.Cu") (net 4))
 (segment (start 222.061 107.975) (end 231.92 107.975) (width 0.3) (layer "B.Cu") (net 4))
 (segment (start 231.92 107.975) (end 233.62 109.675) (width 0.3) (layer "B.Cu") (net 4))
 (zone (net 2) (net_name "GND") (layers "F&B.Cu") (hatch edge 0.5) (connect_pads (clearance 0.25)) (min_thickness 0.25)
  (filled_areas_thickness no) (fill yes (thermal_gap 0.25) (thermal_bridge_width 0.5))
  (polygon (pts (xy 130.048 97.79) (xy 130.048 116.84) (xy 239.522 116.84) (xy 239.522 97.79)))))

